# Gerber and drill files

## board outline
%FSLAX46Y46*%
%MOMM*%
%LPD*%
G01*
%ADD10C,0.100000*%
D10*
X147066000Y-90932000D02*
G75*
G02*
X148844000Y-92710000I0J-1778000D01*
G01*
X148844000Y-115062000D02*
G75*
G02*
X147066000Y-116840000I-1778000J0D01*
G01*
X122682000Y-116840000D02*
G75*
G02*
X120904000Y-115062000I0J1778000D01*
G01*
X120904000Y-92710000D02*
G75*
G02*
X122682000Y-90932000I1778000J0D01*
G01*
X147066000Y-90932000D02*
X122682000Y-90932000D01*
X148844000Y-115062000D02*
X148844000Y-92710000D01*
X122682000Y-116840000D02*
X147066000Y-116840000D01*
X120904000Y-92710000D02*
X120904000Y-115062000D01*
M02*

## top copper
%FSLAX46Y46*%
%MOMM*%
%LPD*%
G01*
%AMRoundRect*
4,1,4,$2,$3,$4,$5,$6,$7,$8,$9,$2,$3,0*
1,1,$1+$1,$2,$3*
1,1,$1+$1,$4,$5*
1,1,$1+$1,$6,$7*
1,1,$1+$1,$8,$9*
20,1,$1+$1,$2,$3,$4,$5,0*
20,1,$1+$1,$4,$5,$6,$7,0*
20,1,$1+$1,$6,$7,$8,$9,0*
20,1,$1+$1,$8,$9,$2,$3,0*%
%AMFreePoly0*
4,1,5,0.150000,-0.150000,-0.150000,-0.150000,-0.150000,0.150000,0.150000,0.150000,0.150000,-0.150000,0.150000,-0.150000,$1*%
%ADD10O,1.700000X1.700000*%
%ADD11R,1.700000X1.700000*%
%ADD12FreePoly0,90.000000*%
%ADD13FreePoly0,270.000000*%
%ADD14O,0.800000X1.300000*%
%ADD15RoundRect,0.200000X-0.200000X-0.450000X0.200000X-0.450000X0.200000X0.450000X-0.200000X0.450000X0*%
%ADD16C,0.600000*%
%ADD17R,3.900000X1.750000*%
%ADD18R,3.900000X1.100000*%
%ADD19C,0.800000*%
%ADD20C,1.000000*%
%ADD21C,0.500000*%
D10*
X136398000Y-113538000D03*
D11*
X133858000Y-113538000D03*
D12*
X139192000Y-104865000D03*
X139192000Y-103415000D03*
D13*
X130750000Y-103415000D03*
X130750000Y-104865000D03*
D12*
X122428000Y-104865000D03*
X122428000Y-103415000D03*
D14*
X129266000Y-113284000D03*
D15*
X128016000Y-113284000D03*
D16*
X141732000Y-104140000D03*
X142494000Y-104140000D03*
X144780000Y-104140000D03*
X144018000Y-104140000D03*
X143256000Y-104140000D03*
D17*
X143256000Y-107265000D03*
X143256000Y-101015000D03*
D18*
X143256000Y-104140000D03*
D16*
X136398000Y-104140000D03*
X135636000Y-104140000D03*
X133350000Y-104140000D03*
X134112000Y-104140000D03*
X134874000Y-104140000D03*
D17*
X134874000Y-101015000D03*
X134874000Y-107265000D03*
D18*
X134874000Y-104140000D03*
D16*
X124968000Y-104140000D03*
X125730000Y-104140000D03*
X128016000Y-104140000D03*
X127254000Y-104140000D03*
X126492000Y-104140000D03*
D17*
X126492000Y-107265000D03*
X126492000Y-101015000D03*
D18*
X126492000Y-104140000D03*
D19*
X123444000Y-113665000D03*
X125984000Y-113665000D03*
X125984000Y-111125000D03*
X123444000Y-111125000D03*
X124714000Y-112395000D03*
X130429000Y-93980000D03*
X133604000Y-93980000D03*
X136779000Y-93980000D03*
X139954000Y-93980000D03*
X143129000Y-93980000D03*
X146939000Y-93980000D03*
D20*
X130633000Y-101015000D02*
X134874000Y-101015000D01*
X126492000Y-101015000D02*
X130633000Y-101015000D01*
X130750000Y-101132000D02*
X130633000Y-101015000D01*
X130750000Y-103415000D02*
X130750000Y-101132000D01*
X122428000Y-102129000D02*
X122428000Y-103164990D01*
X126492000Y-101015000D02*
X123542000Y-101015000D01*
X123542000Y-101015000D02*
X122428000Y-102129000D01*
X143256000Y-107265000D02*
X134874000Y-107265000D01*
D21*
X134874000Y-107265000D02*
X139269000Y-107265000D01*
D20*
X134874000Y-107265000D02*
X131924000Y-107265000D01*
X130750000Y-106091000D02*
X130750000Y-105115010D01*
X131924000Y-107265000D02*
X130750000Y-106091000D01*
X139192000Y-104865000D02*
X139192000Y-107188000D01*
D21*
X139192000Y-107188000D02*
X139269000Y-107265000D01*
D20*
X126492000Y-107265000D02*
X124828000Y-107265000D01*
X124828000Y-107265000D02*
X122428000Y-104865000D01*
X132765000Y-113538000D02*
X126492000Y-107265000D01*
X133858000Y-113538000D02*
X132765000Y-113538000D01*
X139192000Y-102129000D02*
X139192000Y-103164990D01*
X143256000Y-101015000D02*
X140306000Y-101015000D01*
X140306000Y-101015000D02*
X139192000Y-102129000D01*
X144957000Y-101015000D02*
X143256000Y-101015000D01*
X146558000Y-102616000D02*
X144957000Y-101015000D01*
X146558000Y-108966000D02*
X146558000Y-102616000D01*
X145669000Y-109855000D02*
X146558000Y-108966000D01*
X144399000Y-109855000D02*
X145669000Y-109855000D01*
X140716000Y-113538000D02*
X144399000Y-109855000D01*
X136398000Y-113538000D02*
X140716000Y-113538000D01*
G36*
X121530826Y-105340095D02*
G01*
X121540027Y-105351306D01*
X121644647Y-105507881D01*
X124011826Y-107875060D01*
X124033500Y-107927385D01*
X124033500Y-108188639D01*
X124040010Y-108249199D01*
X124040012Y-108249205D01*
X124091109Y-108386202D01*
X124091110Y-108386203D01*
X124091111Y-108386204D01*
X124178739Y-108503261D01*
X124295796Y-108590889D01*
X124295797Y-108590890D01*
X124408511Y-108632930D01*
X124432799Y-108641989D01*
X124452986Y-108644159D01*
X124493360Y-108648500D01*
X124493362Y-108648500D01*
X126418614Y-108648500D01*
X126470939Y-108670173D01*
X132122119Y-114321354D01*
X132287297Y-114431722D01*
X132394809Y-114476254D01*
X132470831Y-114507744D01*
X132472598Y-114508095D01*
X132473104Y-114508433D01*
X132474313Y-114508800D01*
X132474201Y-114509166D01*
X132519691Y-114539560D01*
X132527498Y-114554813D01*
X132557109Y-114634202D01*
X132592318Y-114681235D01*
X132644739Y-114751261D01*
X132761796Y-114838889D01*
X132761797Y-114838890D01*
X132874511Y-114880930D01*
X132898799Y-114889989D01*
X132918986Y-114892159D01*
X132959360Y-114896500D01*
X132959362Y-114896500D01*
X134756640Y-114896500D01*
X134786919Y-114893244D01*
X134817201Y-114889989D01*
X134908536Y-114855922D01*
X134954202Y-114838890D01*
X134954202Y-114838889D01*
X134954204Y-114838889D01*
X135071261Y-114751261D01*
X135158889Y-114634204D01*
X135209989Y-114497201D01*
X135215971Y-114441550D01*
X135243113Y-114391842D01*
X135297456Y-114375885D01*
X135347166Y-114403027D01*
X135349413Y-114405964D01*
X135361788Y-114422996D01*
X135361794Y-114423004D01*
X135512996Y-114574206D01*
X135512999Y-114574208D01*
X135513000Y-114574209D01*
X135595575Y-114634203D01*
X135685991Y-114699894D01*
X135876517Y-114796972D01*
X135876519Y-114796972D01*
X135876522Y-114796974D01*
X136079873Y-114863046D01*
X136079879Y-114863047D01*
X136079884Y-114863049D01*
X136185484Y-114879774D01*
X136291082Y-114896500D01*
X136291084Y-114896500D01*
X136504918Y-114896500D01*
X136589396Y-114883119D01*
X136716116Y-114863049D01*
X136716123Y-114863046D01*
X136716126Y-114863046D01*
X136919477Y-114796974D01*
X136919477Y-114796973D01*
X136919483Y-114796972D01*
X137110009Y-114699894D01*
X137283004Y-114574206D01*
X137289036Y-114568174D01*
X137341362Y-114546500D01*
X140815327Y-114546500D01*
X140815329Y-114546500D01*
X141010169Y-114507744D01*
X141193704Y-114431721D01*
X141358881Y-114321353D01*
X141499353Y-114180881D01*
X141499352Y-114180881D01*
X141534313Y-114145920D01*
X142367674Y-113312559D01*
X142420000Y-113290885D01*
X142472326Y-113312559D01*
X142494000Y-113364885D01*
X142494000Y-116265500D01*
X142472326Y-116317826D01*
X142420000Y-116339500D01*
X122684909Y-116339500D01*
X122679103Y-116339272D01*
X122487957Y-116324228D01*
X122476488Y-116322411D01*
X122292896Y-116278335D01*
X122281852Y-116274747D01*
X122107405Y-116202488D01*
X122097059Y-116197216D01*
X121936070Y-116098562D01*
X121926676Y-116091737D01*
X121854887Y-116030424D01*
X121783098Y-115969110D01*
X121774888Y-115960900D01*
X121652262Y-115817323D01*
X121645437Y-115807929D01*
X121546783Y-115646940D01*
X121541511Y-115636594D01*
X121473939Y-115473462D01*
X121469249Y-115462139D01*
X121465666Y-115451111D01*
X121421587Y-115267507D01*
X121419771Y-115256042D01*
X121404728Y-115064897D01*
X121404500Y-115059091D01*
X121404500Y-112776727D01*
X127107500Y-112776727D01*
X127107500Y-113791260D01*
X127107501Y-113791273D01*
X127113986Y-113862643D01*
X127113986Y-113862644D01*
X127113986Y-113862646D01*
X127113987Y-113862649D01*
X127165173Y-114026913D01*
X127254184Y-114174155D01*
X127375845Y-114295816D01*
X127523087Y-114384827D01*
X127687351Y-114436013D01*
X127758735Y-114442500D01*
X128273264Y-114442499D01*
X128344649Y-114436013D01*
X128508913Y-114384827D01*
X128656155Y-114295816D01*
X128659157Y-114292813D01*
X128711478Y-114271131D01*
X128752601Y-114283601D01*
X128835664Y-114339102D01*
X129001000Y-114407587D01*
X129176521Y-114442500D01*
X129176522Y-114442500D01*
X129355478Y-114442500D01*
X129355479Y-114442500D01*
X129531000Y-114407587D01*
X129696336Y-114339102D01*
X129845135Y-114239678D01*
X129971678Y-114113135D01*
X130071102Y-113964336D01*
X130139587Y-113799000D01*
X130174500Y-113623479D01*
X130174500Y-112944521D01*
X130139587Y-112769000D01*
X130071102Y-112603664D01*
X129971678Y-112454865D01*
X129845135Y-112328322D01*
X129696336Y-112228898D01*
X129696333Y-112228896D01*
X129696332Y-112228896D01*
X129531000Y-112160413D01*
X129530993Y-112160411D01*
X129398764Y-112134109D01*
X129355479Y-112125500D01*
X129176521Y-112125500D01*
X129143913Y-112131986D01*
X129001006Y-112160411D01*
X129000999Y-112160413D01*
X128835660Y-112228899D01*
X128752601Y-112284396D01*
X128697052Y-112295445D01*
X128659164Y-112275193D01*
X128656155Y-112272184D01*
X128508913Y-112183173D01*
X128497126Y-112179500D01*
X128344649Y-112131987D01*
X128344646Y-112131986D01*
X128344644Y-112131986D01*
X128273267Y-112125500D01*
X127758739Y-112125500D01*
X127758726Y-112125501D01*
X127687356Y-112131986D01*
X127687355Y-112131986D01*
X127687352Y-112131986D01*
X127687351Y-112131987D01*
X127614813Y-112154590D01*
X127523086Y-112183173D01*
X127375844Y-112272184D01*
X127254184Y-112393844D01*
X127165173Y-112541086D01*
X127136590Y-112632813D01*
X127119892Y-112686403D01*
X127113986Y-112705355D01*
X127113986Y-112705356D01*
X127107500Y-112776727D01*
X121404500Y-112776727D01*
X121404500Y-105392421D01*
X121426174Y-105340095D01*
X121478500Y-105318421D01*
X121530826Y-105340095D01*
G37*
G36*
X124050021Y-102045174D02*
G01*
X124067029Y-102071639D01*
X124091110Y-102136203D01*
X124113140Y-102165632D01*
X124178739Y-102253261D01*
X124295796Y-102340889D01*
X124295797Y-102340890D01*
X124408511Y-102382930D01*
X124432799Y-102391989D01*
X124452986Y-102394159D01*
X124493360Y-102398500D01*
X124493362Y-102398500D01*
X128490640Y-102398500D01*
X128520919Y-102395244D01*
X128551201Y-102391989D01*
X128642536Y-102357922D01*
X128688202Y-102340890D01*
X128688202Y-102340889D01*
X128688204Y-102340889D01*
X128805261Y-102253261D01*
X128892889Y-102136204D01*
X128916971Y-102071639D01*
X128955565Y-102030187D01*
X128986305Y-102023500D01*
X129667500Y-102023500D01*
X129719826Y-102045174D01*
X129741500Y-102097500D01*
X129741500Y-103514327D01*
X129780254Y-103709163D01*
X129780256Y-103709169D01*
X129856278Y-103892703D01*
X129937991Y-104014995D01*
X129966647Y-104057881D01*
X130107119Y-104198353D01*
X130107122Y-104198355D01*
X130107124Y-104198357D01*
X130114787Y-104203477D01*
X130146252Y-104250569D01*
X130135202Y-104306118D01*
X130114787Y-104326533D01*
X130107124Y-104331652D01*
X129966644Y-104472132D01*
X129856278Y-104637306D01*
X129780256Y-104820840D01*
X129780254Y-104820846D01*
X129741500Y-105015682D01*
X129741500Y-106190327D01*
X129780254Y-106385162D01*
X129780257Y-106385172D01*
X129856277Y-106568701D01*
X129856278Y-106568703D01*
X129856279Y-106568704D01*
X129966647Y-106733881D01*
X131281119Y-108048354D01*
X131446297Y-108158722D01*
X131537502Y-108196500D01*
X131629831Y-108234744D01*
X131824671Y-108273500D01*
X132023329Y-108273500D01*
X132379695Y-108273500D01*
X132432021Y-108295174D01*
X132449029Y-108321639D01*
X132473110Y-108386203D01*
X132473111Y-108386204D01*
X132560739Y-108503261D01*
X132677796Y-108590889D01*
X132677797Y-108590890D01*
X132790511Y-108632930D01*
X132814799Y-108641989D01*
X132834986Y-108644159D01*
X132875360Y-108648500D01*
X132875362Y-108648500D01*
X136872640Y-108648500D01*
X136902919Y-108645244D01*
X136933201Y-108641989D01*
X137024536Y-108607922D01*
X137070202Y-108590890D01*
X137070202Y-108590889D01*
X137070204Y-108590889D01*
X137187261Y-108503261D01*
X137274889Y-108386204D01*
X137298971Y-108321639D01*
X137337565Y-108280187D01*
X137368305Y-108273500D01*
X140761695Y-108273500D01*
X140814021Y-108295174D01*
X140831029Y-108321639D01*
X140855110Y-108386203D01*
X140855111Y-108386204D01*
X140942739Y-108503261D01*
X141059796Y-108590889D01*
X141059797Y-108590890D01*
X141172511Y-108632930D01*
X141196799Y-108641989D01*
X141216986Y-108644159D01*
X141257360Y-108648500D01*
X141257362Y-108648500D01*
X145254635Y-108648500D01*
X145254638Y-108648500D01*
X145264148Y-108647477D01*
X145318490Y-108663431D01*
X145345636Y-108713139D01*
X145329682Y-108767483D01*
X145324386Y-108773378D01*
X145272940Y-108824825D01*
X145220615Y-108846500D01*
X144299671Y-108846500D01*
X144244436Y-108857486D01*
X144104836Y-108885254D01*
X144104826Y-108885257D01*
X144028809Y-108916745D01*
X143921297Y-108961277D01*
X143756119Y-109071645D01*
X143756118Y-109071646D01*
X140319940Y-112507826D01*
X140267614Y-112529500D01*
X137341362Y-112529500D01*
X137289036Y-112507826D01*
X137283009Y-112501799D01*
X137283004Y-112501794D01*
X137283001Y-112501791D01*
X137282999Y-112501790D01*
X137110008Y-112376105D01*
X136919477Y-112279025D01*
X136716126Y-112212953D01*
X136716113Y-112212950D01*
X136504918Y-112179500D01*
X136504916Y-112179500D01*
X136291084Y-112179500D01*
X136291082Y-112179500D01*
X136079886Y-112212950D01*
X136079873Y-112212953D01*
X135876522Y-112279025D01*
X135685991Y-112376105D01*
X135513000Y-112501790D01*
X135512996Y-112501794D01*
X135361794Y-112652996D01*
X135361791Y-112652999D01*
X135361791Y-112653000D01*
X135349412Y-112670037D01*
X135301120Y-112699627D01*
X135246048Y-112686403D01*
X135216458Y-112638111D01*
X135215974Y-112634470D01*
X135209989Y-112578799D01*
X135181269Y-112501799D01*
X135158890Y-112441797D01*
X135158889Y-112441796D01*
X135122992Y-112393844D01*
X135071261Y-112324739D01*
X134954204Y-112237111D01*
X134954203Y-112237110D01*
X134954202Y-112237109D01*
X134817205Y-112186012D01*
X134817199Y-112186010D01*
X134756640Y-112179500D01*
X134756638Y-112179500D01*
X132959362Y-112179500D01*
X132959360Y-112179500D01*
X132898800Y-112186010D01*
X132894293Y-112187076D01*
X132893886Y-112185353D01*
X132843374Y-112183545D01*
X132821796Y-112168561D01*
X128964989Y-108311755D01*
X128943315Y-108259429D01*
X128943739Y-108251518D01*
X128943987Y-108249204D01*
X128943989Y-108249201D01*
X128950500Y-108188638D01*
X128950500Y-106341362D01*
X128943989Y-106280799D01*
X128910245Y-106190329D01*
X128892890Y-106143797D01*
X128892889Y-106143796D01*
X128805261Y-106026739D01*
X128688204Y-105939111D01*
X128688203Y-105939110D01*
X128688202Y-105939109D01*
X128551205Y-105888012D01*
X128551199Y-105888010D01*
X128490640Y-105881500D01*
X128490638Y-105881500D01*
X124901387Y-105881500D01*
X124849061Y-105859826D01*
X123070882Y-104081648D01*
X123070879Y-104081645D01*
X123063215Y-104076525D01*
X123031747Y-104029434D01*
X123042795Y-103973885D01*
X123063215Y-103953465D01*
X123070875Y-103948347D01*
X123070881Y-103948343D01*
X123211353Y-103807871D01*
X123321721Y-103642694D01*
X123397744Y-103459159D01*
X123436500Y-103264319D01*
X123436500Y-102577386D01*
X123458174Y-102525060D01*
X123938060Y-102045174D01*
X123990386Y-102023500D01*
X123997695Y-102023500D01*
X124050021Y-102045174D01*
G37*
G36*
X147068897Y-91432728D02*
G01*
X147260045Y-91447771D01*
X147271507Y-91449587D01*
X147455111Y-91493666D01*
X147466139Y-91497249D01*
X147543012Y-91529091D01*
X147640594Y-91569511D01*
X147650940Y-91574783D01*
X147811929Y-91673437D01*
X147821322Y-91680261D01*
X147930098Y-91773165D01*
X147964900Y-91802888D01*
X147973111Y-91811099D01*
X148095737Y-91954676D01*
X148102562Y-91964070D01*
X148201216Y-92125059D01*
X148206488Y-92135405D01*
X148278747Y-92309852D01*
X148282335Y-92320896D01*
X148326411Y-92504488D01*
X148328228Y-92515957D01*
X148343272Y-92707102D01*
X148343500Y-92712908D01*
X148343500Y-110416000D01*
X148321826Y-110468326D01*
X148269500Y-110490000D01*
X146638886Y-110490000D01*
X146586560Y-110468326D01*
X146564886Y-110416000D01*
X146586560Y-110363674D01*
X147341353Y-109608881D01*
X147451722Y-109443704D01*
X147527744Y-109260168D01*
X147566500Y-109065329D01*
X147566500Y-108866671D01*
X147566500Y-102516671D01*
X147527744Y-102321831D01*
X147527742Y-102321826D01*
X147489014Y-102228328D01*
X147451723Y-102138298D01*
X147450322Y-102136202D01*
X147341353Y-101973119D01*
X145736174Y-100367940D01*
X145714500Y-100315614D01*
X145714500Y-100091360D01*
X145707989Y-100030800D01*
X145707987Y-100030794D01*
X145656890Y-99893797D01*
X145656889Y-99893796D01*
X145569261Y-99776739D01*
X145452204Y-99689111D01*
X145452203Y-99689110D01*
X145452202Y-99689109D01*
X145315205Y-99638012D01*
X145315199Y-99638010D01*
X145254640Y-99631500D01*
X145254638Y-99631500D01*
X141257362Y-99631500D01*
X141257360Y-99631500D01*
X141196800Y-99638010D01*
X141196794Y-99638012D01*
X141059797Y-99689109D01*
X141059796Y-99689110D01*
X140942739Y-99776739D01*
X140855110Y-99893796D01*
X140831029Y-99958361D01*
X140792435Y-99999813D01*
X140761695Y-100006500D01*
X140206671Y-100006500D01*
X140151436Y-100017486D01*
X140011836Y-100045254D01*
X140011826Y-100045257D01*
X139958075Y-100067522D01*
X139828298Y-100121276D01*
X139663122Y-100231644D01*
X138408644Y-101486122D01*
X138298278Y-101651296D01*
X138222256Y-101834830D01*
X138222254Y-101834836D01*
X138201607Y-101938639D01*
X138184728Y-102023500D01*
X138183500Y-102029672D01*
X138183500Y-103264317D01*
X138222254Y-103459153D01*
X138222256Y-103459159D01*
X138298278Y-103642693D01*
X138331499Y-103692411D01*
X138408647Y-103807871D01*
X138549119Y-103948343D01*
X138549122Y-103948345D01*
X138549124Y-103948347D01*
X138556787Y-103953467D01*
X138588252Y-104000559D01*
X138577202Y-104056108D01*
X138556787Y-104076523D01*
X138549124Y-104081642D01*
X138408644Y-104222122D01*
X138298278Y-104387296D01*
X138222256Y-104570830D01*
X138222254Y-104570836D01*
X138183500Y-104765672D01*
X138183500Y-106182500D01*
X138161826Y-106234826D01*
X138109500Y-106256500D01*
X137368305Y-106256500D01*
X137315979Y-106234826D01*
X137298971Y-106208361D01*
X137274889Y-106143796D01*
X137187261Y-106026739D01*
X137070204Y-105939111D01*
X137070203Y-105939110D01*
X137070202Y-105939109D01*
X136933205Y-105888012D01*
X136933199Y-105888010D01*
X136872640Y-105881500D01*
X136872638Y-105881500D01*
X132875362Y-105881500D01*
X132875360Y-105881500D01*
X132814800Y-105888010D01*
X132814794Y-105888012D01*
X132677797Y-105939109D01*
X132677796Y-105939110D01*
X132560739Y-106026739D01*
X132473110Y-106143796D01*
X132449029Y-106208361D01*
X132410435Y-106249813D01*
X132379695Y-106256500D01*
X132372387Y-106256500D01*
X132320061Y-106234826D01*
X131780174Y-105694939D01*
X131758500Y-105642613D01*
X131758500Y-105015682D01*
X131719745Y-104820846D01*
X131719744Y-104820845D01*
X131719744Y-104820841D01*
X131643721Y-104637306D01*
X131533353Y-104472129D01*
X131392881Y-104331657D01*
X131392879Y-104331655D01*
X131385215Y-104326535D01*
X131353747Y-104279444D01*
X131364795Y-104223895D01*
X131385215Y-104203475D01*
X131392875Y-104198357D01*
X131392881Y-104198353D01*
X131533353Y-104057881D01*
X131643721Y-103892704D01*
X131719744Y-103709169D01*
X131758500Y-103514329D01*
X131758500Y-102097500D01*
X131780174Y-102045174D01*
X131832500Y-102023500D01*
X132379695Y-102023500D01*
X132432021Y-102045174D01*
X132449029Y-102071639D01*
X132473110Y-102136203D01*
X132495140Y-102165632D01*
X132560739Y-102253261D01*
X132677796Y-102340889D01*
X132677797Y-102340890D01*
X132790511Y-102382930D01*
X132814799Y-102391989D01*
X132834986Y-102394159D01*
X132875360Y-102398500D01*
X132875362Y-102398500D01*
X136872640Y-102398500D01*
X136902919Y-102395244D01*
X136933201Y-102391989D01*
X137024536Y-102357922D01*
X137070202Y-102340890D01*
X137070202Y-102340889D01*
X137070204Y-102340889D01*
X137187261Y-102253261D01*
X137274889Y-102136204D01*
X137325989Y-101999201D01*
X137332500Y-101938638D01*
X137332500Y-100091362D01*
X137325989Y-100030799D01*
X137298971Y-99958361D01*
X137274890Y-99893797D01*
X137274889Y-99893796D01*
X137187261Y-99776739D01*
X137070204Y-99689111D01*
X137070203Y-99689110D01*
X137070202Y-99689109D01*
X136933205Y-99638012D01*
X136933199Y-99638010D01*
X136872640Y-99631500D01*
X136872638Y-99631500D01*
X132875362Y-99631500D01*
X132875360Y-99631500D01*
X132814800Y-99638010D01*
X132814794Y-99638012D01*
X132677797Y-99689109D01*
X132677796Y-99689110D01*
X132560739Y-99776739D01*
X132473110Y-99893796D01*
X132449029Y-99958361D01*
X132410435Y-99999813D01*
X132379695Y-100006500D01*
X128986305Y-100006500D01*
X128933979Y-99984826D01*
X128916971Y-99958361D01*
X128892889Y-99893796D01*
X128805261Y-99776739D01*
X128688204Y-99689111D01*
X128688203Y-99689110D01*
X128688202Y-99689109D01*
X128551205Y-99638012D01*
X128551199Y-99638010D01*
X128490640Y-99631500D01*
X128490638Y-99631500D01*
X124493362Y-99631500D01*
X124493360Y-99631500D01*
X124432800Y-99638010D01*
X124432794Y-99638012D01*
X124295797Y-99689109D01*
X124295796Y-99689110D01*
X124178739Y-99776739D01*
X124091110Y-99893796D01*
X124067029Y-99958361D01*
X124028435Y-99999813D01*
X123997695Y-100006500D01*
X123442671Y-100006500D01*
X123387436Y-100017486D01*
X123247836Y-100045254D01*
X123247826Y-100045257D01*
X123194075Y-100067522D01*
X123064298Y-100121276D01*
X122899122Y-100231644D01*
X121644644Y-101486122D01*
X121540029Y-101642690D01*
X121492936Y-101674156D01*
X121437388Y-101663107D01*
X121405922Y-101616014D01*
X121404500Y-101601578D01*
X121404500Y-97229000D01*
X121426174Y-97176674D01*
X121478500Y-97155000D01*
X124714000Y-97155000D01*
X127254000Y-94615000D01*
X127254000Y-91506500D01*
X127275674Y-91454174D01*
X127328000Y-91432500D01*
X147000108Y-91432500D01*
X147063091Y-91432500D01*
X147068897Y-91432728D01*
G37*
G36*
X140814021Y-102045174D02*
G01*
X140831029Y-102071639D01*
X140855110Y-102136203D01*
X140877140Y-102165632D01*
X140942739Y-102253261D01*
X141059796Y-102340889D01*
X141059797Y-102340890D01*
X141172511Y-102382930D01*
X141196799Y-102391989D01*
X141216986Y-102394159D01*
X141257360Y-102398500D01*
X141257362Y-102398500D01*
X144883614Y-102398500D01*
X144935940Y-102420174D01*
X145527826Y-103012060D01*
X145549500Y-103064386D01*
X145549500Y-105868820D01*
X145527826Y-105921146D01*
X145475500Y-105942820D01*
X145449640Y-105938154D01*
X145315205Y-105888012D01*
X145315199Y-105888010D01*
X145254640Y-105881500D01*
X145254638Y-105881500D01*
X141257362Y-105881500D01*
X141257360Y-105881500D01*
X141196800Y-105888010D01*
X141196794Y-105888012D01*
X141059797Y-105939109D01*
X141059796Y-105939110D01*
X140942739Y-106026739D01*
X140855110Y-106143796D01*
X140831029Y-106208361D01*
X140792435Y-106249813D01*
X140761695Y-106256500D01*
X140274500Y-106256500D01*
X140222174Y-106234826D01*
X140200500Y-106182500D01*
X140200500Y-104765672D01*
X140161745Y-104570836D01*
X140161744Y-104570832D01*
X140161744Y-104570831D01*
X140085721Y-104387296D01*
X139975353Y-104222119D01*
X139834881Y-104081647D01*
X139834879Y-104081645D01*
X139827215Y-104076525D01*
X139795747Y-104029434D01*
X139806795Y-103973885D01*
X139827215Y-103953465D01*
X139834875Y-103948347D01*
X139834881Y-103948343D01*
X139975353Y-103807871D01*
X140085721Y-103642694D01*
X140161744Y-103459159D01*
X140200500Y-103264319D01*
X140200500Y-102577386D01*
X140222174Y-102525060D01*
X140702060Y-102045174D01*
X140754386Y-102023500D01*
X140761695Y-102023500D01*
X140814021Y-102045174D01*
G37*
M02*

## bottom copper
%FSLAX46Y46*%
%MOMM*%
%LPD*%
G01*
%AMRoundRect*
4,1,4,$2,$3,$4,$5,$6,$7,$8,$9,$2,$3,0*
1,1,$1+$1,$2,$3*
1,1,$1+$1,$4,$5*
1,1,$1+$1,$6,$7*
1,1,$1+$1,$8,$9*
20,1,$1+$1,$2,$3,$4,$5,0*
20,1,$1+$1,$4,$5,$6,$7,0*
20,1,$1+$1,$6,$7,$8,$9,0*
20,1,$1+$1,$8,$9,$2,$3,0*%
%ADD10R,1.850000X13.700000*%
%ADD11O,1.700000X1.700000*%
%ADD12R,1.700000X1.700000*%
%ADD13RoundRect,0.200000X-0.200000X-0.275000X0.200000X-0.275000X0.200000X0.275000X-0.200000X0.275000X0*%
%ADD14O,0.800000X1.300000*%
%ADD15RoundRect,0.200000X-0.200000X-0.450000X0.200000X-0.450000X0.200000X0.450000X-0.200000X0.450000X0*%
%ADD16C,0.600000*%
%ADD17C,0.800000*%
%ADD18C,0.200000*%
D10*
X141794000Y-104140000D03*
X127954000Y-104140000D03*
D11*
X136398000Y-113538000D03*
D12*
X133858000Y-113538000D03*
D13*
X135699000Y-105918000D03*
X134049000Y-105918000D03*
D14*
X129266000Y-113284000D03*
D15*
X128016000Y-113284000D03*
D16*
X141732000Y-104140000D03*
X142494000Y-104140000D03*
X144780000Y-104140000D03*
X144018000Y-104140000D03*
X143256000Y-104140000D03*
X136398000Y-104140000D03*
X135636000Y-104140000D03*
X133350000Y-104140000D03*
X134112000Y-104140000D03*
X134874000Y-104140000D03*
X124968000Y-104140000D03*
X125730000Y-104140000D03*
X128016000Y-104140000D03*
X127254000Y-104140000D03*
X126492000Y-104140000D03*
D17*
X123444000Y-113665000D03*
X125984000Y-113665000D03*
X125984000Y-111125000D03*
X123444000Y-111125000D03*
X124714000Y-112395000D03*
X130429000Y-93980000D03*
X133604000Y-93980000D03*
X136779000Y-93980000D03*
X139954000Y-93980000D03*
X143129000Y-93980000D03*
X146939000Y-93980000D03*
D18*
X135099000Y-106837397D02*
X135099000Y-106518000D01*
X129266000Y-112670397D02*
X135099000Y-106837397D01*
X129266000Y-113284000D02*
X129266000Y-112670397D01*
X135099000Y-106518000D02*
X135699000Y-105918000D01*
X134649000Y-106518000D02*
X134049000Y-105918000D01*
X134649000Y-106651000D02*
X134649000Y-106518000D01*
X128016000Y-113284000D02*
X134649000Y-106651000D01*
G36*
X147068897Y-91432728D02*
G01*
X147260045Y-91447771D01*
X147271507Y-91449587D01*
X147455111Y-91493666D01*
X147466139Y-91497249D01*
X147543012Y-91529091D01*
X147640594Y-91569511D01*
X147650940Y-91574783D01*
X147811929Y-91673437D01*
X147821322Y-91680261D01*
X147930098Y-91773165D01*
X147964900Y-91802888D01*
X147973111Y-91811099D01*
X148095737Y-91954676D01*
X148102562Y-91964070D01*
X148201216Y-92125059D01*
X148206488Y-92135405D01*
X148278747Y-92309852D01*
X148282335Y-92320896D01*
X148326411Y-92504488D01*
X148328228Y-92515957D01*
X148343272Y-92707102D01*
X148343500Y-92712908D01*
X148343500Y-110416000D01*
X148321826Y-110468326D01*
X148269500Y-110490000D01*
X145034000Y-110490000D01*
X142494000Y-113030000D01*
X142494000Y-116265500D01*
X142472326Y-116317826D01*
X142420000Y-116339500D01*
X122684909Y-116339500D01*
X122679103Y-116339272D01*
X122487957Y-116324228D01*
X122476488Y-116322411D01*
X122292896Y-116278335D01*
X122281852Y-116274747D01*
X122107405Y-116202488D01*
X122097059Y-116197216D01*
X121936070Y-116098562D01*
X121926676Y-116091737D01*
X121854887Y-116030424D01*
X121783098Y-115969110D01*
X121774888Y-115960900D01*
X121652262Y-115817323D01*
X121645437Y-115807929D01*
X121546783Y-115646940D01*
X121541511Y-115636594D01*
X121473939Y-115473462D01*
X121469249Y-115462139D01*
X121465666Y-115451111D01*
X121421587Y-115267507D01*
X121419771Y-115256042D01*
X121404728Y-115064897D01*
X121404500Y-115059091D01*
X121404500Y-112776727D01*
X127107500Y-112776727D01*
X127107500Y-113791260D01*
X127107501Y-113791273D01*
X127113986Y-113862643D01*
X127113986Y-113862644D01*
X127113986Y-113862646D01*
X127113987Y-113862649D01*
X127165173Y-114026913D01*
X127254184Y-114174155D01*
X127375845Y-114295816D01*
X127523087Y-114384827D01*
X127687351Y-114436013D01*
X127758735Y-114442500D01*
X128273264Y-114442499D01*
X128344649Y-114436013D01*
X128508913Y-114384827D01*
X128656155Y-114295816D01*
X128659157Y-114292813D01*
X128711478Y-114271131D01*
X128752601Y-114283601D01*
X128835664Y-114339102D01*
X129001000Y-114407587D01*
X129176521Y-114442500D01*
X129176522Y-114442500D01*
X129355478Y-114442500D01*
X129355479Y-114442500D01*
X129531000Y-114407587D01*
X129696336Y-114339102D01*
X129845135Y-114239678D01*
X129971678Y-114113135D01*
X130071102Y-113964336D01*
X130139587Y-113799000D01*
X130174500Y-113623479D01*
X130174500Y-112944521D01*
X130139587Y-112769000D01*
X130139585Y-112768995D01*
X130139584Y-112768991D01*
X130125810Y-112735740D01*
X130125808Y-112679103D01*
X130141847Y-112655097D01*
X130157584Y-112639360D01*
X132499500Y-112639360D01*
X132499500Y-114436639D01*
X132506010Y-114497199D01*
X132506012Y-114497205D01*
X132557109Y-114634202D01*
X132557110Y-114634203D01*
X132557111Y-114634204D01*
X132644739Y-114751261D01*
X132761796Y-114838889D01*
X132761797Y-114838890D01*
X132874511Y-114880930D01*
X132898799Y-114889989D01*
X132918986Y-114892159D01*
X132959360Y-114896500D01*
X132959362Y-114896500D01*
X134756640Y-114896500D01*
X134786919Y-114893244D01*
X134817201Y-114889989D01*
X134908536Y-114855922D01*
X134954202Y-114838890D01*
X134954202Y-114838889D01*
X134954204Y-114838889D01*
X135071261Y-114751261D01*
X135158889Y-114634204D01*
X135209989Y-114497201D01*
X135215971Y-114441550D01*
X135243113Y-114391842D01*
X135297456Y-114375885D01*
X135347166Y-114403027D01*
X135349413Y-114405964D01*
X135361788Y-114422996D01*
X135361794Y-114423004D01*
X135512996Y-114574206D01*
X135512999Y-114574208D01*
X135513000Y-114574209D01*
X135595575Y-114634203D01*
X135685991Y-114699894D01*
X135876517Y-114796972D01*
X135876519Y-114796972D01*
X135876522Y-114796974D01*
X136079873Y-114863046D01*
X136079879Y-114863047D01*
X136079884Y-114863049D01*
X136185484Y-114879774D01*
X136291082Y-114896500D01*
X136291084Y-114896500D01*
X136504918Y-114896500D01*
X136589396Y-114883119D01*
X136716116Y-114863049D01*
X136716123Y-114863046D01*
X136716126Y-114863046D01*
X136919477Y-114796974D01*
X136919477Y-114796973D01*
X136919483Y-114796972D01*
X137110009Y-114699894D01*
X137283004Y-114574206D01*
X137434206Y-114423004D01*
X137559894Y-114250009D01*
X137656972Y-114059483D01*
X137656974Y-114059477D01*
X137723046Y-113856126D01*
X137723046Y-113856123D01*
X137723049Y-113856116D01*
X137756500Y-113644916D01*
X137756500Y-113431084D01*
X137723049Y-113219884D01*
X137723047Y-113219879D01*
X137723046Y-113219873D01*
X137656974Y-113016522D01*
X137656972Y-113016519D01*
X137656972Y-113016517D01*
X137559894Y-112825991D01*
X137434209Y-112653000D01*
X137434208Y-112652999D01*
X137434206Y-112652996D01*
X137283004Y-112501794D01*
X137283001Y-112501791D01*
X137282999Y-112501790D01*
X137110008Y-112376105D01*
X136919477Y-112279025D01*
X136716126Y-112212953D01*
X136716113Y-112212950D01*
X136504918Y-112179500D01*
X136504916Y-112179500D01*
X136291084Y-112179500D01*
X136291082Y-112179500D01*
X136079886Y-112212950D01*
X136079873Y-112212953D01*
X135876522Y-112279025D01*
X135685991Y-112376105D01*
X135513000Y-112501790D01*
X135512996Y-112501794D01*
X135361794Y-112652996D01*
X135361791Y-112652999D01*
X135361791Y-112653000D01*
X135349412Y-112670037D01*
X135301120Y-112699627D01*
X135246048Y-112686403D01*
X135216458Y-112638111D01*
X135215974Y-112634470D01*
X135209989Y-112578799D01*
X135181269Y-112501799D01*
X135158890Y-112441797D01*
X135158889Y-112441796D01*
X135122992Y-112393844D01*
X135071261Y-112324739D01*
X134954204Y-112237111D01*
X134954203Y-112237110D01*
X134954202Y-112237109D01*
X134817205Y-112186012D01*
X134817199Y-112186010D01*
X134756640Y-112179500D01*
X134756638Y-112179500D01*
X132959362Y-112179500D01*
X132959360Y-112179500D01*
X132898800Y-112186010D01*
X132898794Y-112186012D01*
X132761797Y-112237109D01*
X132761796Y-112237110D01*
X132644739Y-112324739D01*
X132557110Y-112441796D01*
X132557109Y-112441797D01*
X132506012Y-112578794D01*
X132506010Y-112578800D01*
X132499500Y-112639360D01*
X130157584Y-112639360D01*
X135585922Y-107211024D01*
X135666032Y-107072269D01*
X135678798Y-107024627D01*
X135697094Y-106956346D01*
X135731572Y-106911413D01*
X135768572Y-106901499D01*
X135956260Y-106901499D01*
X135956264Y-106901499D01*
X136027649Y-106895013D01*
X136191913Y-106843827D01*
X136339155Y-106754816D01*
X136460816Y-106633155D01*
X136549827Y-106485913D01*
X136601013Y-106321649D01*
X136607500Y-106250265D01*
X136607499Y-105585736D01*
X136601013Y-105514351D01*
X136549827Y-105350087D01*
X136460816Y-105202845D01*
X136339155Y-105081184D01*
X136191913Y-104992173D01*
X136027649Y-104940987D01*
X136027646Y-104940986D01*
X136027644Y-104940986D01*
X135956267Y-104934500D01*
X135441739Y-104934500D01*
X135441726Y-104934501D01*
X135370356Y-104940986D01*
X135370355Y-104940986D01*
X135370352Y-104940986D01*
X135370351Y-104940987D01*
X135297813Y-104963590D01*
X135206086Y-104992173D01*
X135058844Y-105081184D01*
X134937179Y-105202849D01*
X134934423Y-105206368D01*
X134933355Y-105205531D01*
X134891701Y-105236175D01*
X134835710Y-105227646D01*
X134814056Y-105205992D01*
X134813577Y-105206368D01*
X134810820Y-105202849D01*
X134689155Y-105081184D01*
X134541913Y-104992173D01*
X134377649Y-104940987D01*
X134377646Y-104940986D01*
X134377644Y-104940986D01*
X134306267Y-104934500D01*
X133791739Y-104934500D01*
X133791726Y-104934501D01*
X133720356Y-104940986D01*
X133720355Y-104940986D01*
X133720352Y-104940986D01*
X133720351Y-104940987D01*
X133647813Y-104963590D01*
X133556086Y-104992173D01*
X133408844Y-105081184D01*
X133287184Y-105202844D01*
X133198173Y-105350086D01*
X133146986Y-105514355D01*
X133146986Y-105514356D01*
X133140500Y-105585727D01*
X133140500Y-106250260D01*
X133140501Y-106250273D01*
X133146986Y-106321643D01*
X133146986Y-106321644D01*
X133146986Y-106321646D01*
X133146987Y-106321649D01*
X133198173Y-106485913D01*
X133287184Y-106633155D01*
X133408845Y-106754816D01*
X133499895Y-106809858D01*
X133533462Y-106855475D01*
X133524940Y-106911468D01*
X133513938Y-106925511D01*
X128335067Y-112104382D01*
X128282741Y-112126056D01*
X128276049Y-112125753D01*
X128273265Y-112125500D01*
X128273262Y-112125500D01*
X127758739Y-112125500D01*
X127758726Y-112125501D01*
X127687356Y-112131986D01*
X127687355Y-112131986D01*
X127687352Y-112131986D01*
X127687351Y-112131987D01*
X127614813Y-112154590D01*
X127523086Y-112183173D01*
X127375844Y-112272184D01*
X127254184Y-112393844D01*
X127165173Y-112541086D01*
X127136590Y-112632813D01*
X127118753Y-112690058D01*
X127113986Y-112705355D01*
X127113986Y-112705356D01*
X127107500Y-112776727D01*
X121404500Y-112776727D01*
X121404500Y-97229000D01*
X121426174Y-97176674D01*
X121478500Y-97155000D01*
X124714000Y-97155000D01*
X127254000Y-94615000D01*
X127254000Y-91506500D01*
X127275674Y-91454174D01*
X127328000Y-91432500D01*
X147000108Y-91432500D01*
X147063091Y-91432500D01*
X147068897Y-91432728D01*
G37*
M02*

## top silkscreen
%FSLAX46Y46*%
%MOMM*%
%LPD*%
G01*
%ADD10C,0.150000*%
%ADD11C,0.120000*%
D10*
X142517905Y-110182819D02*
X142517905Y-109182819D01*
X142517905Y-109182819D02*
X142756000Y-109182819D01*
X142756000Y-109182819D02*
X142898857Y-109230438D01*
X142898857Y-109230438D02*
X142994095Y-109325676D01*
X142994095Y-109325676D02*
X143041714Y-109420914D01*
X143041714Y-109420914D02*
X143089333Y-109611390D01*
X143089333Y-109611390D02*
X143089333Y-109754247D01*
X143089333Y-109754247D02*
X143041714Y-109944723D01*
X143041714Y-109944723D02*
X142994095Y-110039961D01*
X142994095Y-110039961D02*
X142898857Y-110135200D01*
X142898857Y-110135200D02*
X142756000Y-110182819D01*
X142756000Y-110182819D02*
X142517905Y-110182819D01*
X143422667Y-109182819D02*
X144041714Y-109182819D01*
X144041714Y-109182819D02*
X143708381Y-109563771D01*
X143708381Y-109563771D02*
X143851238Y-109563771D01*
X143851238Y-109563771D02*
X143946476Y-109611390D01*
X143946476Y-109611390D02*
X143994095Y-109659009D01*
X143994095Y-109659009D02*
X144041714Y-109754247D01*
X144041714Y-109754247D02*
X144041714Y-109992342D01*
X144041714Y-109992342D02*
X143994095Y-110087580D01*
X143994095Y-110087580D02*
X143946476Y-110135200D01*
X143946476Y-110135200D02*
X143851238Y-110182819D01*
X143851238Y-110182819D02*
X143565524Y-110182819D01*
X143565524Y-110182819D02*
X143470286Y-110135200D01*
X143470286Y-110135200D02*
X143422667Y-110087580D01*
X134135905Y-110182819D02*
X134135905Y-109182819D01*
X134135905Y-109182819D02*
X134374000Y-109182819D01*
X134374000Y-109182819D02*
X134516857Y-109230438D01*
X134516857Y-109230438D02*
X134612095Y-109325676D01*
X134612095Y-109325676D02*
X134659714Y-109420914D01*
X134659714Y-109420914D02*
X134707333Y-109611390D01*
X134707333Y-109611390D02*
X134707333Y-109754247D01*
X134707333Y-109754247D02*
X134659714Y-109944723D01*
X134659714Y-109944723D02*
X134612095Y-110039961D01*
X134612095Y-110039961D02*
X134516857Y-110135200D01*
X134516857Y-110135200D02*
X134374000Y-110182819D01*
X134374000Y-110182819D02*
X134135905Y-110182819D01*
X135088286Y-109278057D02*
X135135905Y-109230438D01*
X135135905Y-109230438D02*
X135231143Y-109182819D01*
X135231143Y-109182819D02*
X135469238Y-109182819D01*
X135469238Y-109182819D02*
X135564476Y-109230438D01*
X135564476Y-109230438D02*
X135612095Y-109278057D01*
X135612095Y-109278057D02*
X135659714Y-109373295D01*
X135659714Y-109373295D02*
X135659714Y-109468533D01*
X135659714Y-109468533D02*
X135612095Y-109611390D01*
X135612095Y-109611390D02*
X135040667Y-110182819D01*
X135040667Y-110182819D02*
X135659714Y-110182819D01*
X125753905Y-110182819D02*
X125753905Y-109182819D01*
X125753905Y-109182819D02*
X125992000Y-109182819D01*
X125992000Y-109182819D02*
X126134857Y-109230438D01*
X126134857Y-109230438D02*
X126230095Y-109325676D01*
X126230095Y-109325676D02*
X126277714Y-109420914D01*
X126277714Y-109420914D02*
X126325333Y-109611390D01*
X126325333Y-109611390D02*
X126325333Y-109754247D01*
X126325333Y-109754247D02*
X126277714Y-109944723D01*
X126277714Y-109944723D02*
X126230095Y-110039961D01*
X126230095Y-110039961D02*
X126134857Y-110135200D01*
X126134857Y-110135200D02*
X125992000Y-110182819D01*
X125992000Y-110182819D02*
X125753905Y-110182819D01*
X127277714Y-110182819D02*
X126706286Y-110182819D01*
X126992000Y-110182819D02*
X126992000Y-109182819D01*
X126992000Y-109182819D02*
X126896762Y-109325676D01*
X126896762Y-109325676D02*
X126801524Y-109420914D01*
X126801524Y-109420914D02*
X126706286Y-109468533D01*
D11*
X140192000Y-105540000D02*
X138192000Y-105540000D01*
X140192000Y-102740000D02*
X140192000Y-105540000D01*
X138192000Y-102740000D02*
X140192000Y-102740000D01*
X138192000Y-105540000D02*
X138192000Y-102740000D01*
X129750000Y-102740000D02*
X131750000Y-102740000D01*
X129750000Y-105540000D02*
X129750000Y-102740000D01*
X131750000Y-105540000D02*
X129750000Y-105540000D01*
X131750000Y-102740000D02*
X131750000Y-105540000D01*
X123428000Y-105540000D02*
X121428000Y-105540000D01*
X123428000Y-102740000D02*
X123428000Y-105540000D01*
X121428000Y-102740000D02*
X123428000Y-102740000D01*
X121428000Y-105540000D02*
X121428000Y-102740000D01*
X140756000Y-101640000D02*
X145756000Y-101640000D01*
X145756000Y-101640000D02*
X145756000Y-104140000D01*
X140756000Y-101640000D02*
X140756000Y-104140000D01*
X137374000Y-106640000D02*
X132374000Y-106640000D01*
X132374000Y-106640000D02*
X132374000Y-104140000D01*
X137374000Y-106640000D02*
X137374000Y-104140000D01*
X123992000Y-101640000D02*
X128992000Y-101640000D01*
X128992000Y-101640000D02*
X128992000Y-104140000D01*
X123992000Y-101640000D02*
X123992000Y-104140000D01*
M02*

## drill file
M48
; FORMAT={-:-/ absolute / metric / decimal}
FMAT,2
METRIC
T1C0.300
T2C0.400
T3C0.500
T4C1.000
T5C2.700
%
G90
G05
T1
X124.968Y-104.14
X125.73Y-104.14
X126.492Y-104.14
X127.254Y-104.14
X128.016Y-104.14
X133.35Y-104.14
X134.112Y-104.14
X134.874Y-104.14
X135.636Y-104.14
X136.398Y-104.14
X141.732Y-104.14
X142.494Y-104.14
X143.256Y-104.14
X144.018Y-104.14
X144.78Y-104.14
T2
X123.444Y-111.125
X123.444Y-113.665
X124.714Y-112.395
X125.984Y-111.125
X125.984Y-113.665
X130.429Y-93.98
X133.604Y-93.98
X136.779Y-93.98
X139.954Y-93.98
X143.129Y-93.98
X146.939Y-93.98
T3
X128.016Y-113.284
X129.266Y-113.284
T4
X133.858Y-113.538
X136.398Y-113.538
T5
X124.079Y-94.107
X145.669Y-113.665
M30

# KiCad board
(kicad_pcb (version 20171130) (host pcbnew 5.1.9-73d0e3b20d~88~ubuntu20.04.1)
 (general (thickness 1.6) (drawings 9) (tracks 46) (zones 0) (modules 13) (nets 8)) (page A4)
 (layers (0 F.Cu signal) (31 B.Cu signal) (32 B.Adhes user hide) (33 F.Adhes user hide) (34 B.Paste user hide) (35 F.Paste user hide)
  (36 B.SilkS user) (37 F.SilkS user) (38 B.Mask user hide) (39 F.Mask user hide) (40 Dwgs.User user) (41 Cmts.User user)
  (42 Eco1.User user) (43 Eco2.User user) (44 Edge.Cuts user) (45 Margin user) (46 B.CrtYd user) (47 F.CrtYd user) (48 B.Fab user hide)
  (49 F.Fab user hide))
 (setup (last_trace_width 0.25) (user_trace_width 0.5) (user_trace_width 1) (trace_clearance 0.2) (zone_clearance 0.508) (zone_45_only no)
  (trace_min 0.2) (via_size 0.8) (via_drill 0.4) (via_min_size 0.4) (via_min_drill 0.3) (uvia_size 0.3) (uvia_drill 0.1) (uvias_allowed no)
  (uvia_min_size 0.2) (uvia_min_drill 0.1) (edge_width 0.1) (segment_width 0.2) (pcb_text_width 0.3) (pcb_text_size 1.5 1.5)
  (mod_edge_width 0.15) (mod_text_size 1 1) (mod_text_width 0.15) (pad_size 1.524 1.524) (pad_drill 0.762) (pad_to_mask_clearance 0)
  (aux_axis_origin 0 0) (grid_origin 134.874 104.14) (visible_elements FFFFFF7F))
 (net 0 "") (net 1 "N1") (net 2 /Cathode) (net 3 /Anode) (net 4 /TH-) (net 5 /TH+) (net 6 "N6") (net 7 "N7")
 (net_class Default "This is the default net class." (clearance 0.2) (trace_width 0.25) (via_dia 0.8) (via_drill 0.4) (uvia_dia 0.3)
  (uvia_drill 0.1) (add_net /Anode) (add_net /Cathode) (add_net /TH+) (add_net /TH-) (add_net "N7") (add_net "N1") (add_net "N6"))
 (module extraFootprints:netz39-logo (layer B.Cu) (at 129.794 93.98 180)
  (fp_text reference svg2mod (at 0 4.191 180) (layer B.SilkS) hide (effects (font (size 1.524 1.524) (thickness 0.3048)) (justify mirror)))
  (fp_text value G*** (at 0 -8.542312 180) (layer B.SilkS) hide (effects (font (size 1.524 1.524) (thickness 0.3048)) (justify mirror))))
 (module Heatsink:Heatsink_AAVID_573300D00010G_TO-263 (layer B.Cu) (at 134.874 104.14 180)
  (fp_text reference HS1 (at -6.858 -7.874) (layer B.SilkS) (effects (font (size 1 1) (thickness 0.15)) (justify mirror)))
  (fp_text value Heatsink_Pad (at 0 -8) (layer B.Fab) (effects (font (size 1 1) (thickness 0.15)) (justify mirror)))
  (pad 1 smd rect (at -6.92 0 180) (size 1.85 13.7) (layers B.Cu B.Paste B.Mask) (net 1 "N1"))
  (pad 1 smd rect (at 6.92 0 180) (size 1.85 13.7) (layers B.Cu B.Paste B.Mask) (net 1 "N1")))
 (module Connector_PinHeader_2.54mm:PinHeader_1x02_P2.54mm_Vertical (layer B.Cu) (at 133.858 113.538 270)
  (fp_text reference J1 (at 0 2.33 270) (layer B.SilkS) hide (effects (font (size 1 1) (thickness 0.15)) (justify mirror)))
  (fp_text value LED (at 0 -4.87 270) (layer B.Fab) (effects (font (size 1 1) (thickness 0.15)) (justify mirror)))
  (pad 2 thru_hole oval (at 0 -2.54 270) (size 1.7 1.7) (drill 1) (layers *.Cu *.Mask) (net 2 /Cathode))
  (pad 1 thru_hole rect (at 0 0 270) (size 1.7 1.7) (drill 1) (layers *.Cu *.Mask) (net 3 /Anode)))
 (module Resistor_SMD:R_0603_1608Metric (layer B.Cu) (at 134.874 105.918)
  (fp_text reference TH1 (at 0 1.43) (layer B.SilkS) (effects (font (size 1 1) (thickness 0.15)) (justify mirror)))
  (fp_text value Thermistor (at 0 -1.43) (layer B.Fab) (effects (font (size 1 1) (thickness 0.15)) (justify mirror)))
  (pad 2 smd roundrect (at 0.825 0) (size 0.8 0.95) (layers B.Cu B.Paste B.Mask) (roundrect_rratio 0.25) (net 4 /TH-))
  (pad 1 smd roundrect (at -0.825 0) (size 0.8 0.95) (layers B.Cu B.Paste B.Mask) (roundrect_rratio 0.25) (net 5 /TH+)))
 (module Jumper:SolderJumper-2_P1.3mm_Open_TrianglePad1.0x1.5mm (layer F.Cu) (at 139.192 104.14 90)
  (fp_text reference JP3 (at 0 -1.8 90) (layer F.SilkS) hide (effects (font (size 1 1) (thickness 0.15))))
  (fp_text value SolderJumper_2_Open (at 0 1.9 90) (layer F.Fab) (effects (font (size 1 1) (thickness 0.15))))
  (fp_line (start -1.4 1) (end -1.4 -1) (layer F.SilkS) (width 0.12))
  (fp_line (start 1.4 1) (end -1.4 1) (layer F.SilkS) (width 0.12))
  (fp_line (start 1.4 -1) (end 1.4 1) (layer F.SilkS) (width 0.12))
  (fp_line (start -1.4 -1) (end 1.4 -1) (layer F.SilkS) (width 0.12))
  (pad 1 smd custom (at -0.725 0 90) (size 0.3 0.3) (layers F.Cu F.Mask) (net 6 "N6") (zone_connect 2)
   (options (clearance outline) (anchor rect)) (primitives))
  (pad 2 smd custom (at 0.725 0 90) (size 0.3 0.3) (layers F.Cu F.Mask) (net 2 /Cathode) (zone_connect 2)
   (options (clearance outline) (anchor rect)) (primitives)))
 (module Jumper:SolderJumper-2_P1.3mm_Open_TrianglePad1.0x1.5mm (layer F.Cu) (at 130.75 104.14 270)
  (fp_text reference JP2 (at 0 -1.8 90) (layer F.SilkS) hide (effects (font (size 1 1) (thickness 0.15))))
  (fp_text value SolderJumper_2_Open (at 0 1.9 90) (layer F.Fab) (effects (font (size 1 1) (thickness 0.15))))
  (fp_line (start -1.4 1) (end -1.4 -1) (layer F.SilkS) (width 0.12))
  (fp_line (start 1.4 1) (end -1.4 1) (layer F.SilkS) (width 0.12))
  (fp_line (start 1.4 -1) (end 1.4 1) (layer F.SilkS) (width 0.12))
  (fp_line (start -1.4 -1) (end 1.4 -1) (layer F.SilkS) (width 0.12))
  (pad 1 smd custom (at -0.725 0 270) (size 0.3 0.3) (layers F.Cu F.Mask) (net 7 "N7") (zone_connect 2)
   (options (clearance outline) (anchor rect)) (primitives))
  (pad 2 smd custom (at 0.725 0 270) (size 0.3 0.3) (layers F.Cu F.Mask) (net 6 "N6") (zone_connect 2)
   (options (clearance outline) (anchor rect)) (primitives)))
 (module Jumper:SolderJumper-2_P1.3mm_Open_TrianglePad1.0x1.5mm (layer F.Cu) (at 122.428 104.14 90)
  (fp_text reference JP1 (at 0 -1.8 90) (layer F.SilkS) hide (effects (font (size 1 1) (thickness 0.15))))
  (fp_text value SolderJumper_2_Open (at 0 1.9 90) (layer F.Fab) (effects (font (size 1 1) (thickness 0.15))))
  (fp_line (start -1.4 1) (end -1.4 -1) (layer F.SilkS) (width 0.12))
  (fp_line (start 1.4 1) (end -1.4 1) (layer F.SilkS) (width 0.12))
  (fp_line (start 1.4 -1) (end 1.4 1) (layer F.SilkS) (width 0.12))
  (fp_line (start -1.4 -1) (end 1.4 -1) (layer F.SilkS) (width 0.12))
  (pad 1 smd custom (at -0.725 0 90) (size 0.3 0.3) (layers F.Cu F.Mask) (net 3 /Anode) (zone_connect 2)
   (options (clearance outline) (anchor rect)) (primitives))
  (pad 2 smd custom (at 0.725 0 90) (size 0.3 0.3) (layers F.Cu F.Mask) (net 7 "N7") (zone_connect 2)
   (options (clearance outline) (anchor rect)) (primitives)))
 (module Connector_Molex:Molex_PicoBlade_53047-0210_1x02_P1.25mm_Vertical (layer B.Cu) (at 128.016 113.284)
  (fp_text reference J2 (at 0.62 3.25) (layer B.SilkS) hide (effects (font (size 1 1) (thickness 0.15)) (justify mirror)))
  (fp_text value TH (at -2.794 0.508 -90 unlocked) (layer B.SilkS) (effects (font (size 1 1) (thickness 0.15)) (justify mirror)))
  (pad 2 thru_hole oval (at 1.25 0) (size 0.8 1.3) (drill 0.5) (layers *.Cu *.Mask) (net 4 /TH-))
  (pad 1 thru_hole roundrect (at 0 0) (size 0.8 1.3) (drill 0.5) (layers *.Cu *.Mask) (roundrect_rratio 0.25) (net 5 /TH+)))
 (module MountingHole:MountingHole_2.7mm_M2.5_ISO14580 (layer F.Cu) (at 145.669 113.665)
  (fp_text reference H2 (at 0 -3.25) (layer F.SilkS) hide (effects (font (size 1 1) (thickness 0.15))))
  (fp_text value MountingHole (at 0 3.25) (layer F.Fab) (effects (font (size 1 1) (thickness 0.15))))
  (pad 1 np_thru_hole circle (at 0 0) (size 2.7 2.7) (drill 2.7) (layers *.Cu *.Mask)))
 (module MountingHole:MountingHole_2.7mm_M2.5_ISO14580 (layer F.Cu) (at 124.079 94.107)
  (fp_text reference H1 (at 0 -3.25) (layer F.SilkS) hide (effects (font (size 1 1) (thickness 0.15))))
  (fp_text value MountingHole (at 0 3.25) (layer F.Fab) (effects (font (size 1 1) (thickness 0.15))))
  (pad 1 np_thru_hole circle (at 0 0) (size 2.7 2.7) (drill 2.7) (layers *.Cu *.Mask)))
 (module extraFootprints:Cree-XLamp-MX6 (layer F.Cu) (at 143.256 104.14 90)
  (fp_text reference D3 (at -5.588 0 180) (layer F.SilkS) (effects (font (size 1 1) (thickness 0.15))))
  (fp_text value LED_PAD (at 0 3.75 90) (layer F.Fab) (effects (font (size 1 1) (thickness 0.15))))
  (fp_line (start 2.5 -2.5) (end 2.5 2.5) (layer F.SilkS) (width 0.12))
  (fp_line (start 2.5 2.5) (end 0 2.5) (layer F.SilkS) (width 0.12))
  (fp_line (start 2.5 -2.5) (end 0 -2.5) (layer F.SilkS) (width 0.12))
  (pad 3 thru_hole circle (at 0 -1.524 90) (size 0.6 0.6) (drill 0.3) (layers *.Cu *.Mask) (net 1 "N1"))
  (pad 3 thru_hole circle (at 0 -0.762 90) (size 0.6 0.6) (drill 0.3) (layers *.Cu *.Mask) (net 1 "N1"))
  (pad 3 thru_hole circle (at 0 1.524 90) (size 0.6 0.6) (drill 0.3) (layers *.Cu *.Mask) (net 1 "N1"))
  (pad 3 thru_hole circle (at 0 0.762 90) (size 0.6 0.6) (drill 0.3) (layers *.Cu *.Mask) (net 1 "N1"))
  (pad 3 thru_hole circle (at 0 0 90) (size 0.6 0.6) (drill 0.3) (layers *.Cu *.Mask) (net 1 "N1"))
  (pad 2 smd rect (at -3.125 0 90) (size 1.75 3.9) (layers F.Cu F.Paste F.Mask) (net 6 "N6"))
  (pad 1 smd rect (at 3.125 0 90) (size 1.75 3.9) (layers F.Cu F.Paste F.Mask) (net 2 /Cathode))
  (pad 3 smd rect (at 0 0 90) (size 1.1 3.9) (layers F.Cu F.Paste F.Mask) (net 1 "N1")))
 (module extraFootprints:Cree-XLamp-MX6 (layer F.Cu) (at 134.874 104.14 270)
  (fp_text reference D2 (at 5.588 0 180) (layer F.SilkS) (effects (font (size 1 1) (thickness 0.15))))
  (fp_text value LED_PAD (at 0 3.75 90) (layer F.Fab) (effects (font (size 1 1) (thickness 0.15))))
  (fp_line (start 2.5 -2.5) (end 2.5 2.5) (layer F.SilkS) (width 0.12))
  (fp_line (start 2.5 2.5) (end 0 2.5) (layer F.SilkS) (width 0.12))
  (fp_line (start 2.5 -2.5) (end 0 -2.5) (layer F.SilkS) (width 0.12))
  (pad 3 thru_hole circle (at 0 -1.524 270) (size 0.6 0.6) (drill 0.3) (layers *.Cu *.Mask) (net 1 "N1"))
  (pad 3 thru_hole circle (at 0 -0.762 270) (size 0.6 0.6) (drill 0.3) (layers *.Cu *.Mask) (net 1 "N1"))
  (pad 3 thru_hole circle (at 0 1.524 270) (size 0.6 0.6) (drill 0.3) (layers *.Cu *.Mask) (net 1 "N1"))
  (pad 3 thru_hole circle (at 0 0.762 270) (size 0.6 0.6) (drill 0.3) (layers *.Cu *.Mask) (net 1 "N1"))
  (pad 3 thru_hole circle (at 0 0 270) (size 0.6 0.6) (drill 0.3) (layers *.Cu *.Mask) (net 1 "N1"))
  (pad 2 smd rect (at -3.125 0 270) (size 1.75 3.9) (layers F.Cu F.Paste F.Mask) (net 7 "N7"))
  (pad 1 smd rect (at 3.125 0 270) (size 1.75 3.9) (layers F.Cu F.Paste F.Mask) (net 6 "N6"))
  (pad 3 smd rect (at 0 0 270) (size 1.1 3.9) (layers F.Cu F.Paste F.Mask) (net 1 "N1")))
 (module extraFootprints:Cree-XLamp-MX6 (layer F.Cu) (at 126.492 104.14 90)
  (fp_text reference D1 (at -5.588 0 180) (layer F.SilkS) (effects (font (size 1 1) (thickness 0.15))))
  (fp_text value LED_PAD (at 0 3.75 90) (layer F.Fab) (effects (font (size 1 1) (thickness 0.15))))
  (fp_line (start 2.5 -2.5) (end 2.5 2.5) (layer F.SilkS) (width 0.12))
  (fp_line (start 2.5 2.5) (end 0 2.5) (layer F.SilkS) (width 0.12))
  (fp_line (start 2.5 -2.5) (end 0 -2.5) (layer F.SilkS) (width 0.12))
  (pad 3 thru_hole circle (at 0 -1.524 90) (size 0.6 0.6) (drill 0.3) (layers *.Cu *.Mask) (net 1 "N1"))
  (pad 3 thru_hole circle (at 0 -0.762 90) (size 0.6 0.6) (drill 0.3) (layers *.Cu *.Mask) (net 1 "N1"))
  (pad 3 thru_hole circle (at 0 1.524 90) (size 0.6 0.6) (drill 0.3) (layers *.Cu *.Mask) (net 1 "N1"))
  (pad 3 thru_hole circle (at 0 0.762 90) (size 0.6 0.6) (drill 0.3) (layers *.Cu *.Mask) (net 1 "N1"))
  (pad 3 thru_hole circle (at 0 0 90) (size 0.6 0.6) (drill 0.3) (layers *.Cu *.Mask) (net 1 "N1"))
  (pad 2 smd rect (at -3.125 0 90) (size 1.75 3.9) (layers F.Cu F.Paste F.Mask) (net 3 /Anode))
  (pad 1 smd rect (at 3.125 0 90) (size 1.75 3.9) (layers F.Cu F.Paste F.Mask) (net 7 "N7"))
  (pad 3 smd rect (at 0 0 90) (size 1.1 3.9) (layers F.Cu F.Paste F.Mask) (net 1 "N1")))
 (gr_arc (start 147.066 92.71) (end 148.844 92.71) (angle -90) (layer Edge.Cuts) (width 0.1))
 (gr_arc (start 147.066 115.062) (end 147.066 116.84) (angle -90) (layer Edge.Cuts) (width 0.1))
 (gr_arc (start 122.682 115.062) (end 120.904 115.062) (angle -90) (layer Edge.Cuts) (width 0.1))
 (gr_arc (start 122.682 92.71) (end 122.682 90.932) (angle -90) (layer Edge.Cuts) (width 0.1))
 (gr_line (start 147.066 90.932) (end 122.682 90.932) (layer Edge.Cuts) (width 0.1))
 (gr_line (start 148.844 115.062) (end 148.844 92.71) (layer Edge.Cuts) (width 0.1))
 (gr_line (start 122.682 116.84) (end 147.066 116.84) (layer Edge.Cuts) (width 0.1))
 (gr_line (start 120.904 92.71) (end 120.904 115.062) (layer Edge.Cuts) (width 0.1))
 (via (at 123.444 113.665) (size 0.8) (drill 0.4) (layers F.Cu B.Cu) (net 1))
 (via (at 125.984 113.665) (size 0.8) (drill 0.4) (layers F.Cu B.Cu) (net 1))
 (via (at 125.984 111.125) (size 0.8) (drill 0.4) (layers F.Cu B.Cu) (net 1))
 (via (at 123.444 111.125) (size 0.8) (drill 0.4) (layers F.Cu B.Cu) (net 1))
 (via (at 124.714 112.395) (size 0.8) (drill 0.4) (layers F.Cu B.Cu) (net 1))
 (via (at 130.429 93.98) (size 0.8) (drill 0.4) (layers F.Cu B.Cu) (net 1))
 (via (at 133.604 93.98) (size 0.8) (drill 0.4) (layers F.Cu B.Cu) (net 1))
 (via (at 136.779 93.98) (size 0.8) (drill 0.4) (layers F.Cu B.Cu) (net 1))
 (via (at 139.954 93.98) (size 0.8) (drill 0.4) (layers F.Cu B.Cu) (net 1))
 (via (at 143.129 93.98) (size 0.8) (drill 0.4) (layers F.Cu B.Cu) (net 1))
 (via (at 146.939 93.98) (size 0.8) (drill 0.4) (layers F.Cu B.Cu) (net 1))
 (segment (start 130.633 101.015) (end 134.874 101.015) (width 1) (layer F.Cu) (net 7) (status 20))
 (segment (start 126.492 101.015) (end 130.633 101.015) (width 1) (layer F.Cu) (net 7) (status 10))
 (segment (start 130.75 101.132) (end 130.633 101.015) (width 1) (layer F.Cu) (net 7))
 (segment (start 130.75 103.415) (end 130.75 101.132) (width 1) (layer F.Cu) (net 7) (status 10))
 (segment (start 122.428 102.129) (end 122.428 103.16499) (width 1) (layer F.Cu) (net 7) (status 20))
 (segment (start 126.492 101.015) (end 123.542 101.015) (width 1) (layer F.Cu) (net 7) (status 10))
 (segment (start 123.542 101.015) (end 122.428 102.129) (width 1) (layer F.Cu) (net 7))
 (segment (start 143.256 107.265) (end 134.874 107.265) (width 1) (layer F.Cu) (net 6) (status 30))
 (segment (start 134.874 107.265) (end 139.269 107.265) (width 0.5) (layer F.Cu) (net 6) (status 10))
 (segment (start 134.874 107.265) (end 131.924 107.265) (width 1) (layer F.Cu) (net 6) (status 10))
 (segment (start 130.75 106.091) (end 130.75 105.11501) (width 1) (layer F.Cu) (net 6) (status 20))
 (segment (start 131.924 107.265) (end 130.75 106.091) (width 1) (layer F.Cu) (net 6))
 (segment (start 139.192 104.865) (end 139.192 107.188) (width 1) (layer F.Cu) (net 6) (status 10))
 (segment (start 139.192 107.188) (end 139.269 107.265) (width 0.5) (layer F.Cu) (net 6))
 (segment (start 126.492 107.265) (end 124.828 107.265) (width 1) (layer F.Cu) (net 3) (status 30))
 (segment (start 124.828 107.265) (end 122.428 104.865) (width 1) (layer F.Cu) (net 3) (status 30))
 (segment (start 132.765 113.538) (end 126.492 107.265) (width 1) (layer F.Cu) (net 3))
 (segment (start 133.858 113.538) (end 132.765 113.538) (width 1) (layer F.Cu) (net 3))
 (segment (start 139.192 102.129) (end 139.192 103.16499) (width 1) (layer F.Cu) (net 2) (status 20))
 (segment (start 143.256 101.015) (end 140.306 101.015) (width 1) (layer F.Cu) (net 2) (status 10))
 (segment (start 140.306 101.015) (end 139.192 102.129) (width 1) (layer F.Cu) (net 2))
 (segment (start 144.957 101.015) (end 143.256 101.015) (width 1) (layer F.Cu) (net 2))
 (segment (start 146.558 102.616) (end 144.957 101.015) (width 1) (layer F.Cu) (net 2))
 (segment (start 146.558 108.966) (end 146.558 102.616) (width 1) (layer F.Cu) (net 2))
 (segment (start 145.669 109.855) (end 146.558 108.966) (width 1) (layer F.Cu) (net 2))
 (segment (start 144.399 109.855) (end 145.669 109.855) (width 1) (layer F.Cu) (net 2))
 (segment (start 140.716 113.538) (end 144.399 109.855) (width 1) (layer F.Cu) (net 2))
 (segment (start 136.398 113.538) (end 140.716 113.538) (width 1) (layer F.Cu) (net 2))
 (segment (start 135.099 106.837397) (end 135.099 106.518) (width 0.2) (layer B.Cu) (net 4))
 (segment (start 129.266 112.670397) (end 135.099 106.837397) (width 0.2) (layer B.Cu) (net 4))
 (segment (start 129.266 113.284) (end 129.266 112.670397) (width 0.2) (layer B.Cu) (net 4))
 (segment (start 135.099 106.518) (end 135.699 105.918) (width 0.2) (layer B.Cu) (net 4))
 (segment (start 134.649 106.518) (end 134.049 105.918) (width 0.2) (layer B.Cu) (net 5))
 (segment (start 134.649 106.651) (end 134.649 106.518) (width 0.2) (layer B.Cu) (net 5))
 (segment (start 128.016 113.284) (end 134.649 106.651) (width 0.2) (layer B.Cu) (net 5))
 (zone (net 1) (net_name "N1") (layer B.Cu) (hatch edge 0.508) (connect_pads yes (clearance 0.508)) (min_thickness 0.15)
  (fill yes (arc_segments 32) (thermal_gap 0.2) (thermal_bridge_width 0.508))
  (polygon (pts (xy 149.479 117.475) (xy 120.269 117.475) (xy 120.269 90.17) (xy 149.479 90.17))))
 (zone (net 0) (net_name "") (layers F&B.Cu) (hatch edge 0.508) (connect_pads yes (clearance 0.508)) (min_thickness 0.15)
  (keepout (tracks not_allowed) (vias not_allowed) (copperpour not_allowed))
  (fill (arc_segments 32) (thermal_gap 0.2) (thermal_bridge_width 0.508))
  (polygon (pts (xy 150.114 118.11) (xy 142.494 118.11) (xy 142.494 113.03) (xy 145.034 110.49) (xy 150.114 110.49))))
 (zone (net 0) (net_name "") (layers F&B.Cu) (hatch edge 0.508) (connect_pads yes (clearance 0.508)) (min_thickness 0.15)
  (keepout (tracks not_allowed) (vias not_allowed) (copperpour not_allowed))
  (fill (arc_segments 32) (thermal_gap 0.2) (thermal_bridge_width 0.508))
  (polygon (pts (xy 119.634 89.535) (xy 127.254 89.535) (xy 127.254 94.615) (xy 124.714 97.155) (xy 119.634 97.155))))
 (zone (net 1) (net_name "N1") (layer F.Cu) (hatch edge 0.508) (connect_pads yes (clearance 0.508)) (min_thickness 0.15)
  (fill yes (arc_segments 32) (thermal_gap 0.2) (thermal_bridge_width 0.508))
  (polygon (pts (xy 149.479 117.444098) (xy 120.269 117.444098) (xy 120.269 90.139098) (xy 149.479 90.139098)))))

